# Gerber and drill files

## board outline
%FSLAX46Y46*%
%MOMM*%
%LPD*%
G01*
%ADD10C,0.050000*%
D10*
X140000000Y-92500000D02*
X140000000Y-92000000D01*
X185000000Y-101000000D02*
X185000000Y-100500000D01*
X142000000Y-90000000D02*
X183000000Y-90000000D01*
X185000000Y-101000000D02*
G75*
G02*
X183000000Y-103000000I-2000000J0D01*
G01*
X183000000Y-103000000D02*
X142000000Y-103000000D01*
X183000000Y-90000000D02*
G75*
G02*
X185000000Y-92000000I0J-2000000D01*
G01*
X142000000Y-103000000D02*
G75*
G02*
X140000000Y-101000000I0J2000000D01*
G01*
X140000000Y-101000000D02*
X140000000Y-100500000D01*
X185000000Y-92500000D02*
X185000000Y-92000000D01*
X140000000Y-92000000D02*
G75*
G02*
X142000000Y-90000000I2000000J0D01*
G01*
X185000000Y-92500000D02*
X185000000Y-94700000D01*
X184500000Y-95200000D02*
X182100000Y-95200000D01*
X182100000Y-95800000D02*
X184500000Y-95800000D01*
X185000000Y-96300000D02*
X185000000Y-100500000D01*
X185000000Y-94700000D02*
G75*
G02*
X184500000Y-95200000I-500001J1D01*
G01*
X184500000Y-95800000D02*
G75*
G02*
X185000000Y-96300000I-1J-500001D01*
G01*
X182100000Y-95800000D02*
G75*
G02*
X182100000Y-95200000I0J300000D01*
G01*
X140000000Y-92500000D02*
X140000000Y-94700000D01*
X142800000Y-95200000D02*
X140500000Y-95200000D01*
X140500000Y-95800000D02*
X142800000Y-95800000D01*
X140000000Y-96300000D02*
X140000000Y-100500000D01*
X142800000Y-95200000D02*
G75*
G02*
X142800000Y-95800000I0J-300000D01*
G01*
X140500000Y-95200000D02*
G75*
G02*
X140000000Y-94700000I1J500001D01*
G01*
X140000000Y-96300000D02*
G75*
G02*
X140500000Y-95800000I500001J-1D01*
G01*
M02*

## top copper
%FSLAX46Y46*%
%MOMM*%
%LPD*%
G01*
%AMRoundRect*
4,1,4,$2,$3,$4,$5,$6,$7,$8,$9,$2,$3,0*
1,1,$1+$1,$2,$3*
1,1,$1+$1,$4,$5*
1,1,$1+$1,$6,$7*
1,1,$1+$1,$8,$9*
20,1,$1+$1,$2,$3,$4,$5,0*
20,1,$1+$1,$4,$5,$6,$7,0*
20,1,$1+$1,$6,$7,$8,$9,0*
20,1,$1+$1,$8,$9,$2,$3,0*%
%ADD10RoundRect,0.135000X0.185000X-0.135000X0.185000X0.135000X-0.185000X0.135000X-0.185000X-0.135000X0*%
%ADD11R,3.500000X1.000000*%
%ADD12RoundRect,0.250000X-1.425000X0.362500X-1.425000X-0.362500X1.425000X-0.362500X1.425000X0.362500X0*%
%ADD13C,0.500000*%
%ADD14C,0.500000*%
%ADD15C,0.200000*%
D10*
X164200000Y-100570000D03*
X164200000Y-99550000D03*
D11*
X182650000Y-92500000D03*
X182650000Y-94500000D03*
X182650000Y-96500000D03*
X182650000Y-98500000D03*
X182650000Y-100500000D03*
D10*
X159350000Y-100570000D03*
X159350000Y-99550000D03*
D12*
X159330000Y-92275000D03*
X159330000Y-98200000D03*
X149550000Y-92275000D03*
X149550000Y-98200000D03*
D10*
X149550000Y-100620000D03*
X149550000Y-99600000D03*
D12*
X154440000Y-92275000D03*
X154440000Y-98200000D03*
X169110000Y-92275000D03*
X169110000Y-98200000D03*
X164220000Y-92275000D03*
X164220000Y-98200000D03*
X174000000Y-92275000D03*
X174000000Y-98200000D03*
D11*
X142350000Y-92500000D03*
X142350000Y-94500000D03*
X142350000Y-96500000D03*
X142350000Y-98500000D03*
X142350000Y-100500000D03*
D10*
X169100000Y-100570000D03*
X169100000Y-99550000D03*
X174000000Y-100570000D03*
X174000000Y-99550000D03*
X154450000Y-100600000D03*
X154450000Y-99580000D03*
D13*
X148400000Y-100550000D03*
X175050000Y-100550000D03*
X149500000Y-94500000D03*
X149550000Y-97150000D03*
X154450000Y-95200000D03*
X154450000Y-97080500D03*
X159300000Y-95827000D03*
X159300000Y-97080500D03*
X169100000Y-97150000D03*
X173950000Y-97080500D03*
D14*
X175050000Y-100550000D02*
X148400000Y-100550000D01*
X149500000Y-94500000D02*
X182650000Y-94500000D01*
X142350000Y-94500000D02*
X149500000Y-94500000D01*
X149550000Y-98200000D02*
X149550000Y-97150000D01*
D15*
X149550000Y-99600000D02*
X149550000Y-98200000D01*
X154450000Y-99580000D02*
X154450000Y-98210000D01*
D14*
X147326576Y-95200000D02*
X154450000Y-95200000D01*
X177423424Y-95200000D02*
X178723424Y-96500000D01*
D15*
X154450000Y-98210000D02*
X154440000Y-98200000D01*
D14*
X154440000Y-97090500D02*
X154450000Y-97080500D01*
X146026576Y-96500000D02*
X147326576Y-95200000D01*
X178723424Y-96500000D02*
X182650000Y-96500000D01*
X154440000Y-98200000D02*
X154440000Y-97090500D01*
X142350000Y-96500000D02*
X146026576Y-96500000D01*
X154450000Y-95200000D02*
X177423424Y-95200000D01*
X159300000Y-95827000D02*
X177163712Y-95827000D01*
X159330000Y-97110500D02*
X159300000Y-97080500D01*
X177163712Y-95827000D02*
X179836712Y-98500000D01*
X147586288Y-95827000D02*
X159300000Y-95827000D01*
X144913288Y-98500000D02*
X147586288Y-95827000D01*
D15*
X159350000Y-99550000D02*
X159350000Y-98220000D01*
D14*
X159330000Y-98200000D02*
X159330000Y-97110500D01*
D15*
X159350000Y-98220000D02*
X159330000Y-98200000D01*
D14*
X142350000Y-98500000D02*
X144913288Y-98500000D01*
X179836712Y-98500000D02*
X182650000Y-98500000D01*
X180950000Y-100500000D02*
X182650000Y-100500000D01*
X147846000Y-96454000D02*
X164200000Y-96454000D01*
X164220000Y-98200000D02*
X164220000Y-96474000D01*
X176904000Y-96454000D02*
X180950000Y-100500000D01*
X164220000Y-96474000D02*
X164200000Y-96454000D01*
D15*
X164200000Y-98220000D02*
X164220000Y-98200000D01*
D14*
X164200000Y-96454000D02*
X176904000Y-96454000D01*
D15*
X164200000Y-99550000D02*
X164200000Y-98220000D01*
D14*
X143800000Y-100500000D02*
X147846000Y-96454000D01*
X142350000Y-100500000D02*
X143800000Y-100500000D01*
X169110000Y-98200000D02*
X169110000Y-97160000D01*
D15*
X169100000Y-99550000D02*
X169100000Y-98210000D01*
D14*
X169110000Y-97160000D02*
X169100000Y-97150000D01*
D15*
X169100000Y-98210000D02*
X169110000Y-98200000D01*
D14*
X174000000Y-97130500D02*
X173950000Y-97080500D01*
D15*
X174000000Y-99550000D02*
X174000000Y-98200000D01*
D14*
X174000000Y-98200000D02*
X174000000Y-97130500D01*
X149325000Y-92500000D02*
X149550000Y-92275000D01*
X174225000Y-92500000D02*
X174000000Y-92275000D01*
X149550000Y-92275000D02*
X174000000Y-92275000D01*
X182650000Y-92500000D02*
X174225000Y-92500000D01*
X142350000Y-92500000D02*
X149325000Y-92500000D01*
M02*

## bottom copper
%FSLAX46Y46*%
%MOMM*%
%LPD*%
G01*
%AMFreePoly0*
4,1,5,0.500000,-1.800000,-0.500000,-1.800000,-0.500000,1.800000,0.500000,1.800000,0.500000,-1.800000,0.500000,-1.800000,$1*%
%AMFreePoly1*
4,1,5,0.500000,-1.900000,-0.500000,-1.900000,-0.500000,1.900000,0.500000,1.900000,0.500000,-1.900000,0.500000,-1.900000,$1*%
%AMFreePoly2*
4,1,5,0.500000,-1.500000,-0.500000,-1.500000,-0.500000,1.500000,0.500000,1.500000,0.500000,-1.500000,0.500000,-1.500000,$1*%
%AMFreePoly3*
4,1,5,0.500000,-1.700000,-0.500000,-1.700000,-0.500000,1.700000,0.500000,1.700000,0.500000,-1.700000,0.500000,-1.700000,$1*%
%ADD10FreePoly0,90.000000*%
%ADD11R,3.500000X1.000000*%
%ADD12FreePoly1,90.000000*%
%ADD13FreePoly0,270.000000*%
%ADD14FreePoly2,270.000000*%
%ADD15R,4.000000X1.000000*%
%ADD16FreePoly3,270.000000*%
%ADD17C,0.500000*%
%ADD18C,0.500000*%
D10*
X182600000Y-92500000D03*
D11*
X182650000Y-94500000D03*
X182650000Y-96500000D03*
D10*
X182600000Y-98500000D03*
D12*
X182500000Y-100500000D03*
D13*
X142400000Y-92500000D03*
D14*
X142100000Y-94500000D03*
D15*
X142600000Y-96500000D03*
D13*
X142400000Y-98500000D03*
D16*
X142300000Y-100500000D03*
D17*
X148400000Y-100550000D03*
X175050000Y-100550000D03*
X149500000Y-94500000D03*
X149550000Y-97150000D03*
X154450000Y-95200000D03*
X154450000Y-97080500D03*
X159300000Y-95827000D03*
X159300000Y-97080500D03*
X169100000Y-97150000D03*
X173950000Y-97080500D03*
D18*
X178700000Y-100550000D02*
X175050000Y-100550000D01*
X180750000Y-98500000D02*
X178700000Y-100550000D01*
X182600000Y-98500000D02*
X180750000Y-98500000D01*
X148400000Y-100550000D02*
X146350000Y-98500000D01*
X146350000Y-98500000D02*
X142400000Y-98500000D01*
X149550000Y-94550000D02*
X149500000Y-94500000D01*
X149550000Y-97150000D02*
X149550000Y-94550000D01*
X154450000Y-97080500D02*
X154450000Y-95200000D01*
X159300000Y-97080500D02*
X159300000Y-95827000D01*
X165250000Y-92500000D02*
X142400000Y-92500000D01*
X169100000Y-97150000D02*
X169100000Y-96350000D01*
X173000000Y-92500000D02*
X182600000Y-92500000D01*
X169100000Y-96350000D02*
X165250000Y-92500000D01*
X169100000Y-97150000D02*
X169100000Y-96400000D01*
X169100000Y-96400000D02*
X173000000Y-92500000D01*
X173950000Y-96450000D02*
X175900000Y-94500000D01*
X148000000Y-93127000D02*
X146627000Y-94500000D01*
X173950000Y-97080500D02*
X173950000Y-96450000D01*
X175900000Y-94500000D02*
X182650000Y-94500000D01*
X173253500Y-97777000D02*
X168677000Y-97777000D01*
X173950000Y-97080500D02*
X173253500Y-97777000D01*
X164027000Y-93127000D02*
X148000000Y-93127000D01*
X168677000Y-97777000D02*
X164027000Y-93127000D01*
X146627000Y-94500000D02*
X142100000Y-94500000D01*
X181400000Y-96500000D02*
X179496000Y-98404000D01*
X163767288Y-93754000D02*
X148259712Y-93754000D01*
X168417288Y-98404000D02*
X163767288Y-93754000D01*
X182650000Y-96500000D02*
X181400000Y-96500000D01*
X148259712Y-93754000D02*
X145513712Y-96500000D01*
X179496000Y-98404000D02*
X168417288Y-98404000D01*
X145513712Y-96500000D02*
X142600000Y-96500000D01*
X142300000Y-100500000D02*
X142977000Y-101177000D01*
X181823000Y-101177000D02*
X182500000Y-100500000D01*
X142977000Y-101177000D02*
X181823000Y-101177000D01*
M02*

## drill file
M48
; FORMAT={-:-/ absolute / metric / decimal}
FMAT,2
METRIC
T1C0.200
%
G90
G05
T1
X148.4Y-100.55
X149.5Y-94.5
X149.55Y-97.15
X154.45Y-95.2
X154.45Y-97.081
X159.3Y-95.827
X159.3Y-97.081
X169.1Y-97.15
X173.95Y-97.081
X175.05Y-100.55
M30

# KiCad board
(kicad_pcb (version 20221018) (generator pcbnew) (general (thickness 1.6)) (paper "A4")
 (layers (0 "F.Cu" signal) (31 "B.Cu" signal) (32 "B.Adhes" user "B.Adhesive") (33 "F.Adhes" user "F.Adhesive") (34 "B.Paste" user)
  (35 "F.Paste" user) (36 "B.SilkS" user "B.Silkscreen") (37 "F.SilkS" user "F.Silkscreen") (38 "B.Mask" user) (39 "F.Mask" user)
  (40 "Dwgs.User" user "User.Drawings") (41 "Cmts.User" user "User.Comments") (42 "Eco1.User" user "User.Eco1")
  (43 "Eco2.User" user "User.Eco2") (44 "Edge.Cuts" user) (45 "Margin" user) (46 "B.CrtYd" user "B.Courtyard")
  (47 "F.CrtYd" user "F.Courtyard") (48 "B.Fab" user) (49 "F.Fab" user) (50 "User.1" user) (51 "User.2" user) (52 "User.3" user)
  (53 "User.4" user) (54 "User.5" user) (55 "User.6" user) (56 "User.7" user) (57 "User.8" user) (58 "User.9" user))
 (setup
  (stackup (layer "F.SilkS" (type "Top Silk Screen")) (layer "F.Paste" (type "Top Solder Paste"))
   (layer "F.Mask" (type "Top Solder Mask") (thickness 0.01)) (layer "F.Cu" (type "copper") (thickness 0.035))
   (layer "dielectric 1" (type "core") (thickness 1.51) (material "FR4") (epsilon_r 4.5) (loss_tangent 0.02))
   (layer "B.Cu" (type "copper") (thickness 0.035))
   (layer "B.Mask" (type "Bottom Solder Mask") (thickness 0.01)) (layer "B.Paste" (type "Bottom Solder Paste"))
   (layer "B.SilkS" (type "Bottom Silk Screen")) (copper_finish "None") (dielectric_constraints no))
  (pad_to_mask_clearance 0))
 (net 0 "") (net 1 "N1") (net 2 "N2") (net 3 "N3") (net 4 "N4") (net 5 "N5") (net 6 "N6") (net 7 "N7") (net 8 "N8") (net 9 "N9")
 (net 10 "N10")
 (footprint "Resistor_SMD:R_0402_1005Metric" (layer "F.Cu") (at 164.2 100.06 90)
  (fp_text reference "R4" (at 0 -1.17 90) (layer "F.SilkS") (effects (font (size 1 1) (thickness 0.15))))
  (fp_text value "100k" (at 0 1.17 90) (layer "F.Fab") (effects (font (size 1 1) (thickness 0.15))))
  (pad "1" smd roundrect (at -0.51 0 90) (size 0.54 0.64) (layers "F.Cu" "F.Paste" "F.Mask") (roundrect_rratio 0.25) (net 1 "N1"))
  (pad "2" smd roundrect (at 0.51 0 90) (size 0.54 0.64) (layers "F.Cu" "F.Paste" "F.Mask") (roundrect_rratio 0.25) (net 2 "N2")))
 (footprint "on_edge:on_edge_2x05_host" (layer "F.Cu") (at 185 96.5 -90)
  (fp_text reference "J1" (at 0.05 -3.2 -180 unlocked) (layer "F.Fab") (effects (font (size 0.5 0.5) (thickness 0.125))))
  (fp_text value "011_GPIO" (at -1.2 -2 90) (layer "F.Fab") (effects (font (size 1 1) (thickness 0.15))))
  (fp_line (start -4 0) (end -1.8 0) (stroke (width 0.05) (type solid)) (layer "Edge.Cuts"))
  (fp_line (start -1.3 0.5) (end -1.3 2.9) (stroke (width 0.05) (type solid)) (layer "Edge.Cuts"))
  (fp_line (start -0.7 2.9) (end -0.7 0.5) (stroke (width 0.05) (type solid)) (layer "Edge.Cuts"))
  (fp_line (start -0.2 0) (end 4 0) (stroke (width 0.05) (type solid)) (layer "Edge.Cuts"))
  (fp_arc (start -1.8 0) (mid -1.446447 0.146447) (end -1.3 0.5) (stroke (width 0.05) (type solid)) (layer "Edge.Cuts"))
  (fp_arc (start -0.7 0.5) (mid -0.553553 0.146447) (end -0.2 0) (stroke (width 0.05) (type solid)) (layer "Edge.Cuts"))
  (fp_arc (start -0.7 2.9) (mid -1 3.2) (end -1.3 2.9) (stroke (width 0.05) (type solid)) (layer "Edge.Cuts"))
  (pad "1" smd rect (at -4 2.35 270) (size 1 3.5) (layers "F.Cu" "F.Mask") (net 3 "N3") (zone_connect 0))
  (pad "2" smd rect (at -2 2.35 270) (size 1 3.5) (layers "F.Cu" "F.Mask") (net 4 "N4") (zone_connect 0))
  (pad "3" smd rect (at 0 2.35 270) (size 1 3.5) (layers "F.Cu" "F.Mask") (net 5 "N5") (zone_connect 0))
  (pad "4" smd rect (at 2 2.35 270) (size 1 3.5) (layers "F.Cu" "F.Mask") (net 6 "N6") (zone_connect 0))
  (pad "5" smd rect (at 4 2.35 270) (size 1 3.5) (layers "F.Cu" "F.Mask") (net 2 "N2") (zone_connect 0))
  (pad "6" smd custom (at -4 2.4 90) (size 1 3.6) (layers "B.Cu" "B.Mask") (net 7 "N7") (zone_connect 0)
   (options (clearance outline) (anchor rect)) (primitives))
  (pad "7" smd rect (at -2 2.35 90) (size 1 3.5) (layers "B.Cu" "B.Mask") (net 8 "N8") (zone_connect 0))
  (pad "8" smd rect (at 0 2.35 90) (size 1 3.5) (layers "B.Cu" "B.Mask") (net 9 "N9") (zone_connect 0))
  (pad "9" smd custom (at 2 2.4 90) (size 1 3.6) (layers "B.Cu" "B.Mask") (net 1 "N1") (zone_connect 0)
   (options (clearance outline) (anchor rect)) (primitives))
  (pad "10" smd custom (at 4 2.5 90) (size 1 3.8) (layers "B.Cu" "B.Mask") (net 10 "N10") (zone_connect 0)
   (options (clearance outline) (anchor rect)) (primitives))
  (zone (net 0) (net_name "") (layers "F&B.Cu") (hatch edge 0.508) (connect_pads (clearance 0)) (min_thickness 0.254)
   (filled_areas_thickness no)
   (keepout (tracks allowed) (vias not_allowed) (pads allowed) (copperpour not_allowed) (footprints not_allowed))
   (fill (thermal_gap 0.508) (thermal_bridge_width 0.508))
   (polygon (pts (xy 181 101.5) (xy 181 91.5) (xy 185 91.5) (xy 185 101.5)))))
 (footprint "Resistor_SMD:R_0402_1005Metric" (layer "F.Cu") (at 159.35 100.06 90)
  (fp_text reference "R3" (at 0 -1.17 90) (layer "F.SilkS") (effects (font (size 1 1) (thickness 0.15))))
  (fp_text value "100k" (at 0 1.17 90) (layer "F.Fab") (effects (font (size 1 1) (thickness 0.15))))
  (pad "1" smd roundrect (at -0.51 0 90) (size 0.54 0.64) (layers "F.Cu" "F.Paste" "F.Mask") (roundrect_rratio 0.25) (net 1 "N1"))
  (pad "2" smd roundrect (at 0.51 0 90) (size 0.54 0.64) (layers "F.Cu" "F.Paste" "F.Mask") (roundrect_rratio 0.25) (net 6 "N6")))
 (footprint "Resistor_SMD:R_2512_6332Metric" (layer "F.Cu") (at 159.33 95.2375 -90)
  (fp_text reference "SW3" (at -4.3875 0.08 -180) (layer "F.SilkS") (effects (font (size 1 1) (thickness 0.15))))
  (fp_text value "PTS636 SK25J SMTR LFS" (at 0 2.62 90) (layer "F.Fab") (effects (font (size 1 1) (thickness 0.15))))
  (pad "1" smd roundrect (at -2.9625 0 270) (size 1.225 3.35) (layers "F.Cu" "F.Paste" "F.Mask") (roundrect_rratio 0.2040816327)
   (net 3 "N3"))
  (pad "2" smd roundrect (at 2.9625 0 270) (size 1.225 3.35) (layers "F.Cu" "F.Paste" "F.Mask") (roundrect_rratio 0.2040816327) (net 6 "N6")))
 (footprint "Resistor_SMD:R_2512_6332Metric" (layer "F.Cu") (at 149.55 95.2375 -90)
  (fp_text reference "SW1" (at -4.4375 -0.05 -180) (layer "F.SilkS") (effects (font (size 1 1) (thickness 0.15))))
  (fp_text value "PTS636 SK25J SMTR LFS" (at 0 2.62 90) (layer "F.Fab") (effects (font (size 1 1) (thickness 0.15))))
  (pad "1" smd roundrect (at -2.9625 0 270) (size 1.225 3.35) (layers "F.Cu" "F.Paste" "F.Mask") (roundrect_rratio 0.2040816327)
   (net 3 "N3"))
  (pad "2" smd roundrect (at 2.9625 0 270) (size 1.225 3.35) (layers "F.Cu" "F.Paste" "F.Mask") (roundrect_rratio 0.2040816327) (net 4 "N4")))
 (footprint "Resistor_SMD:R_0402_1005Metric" (layer "F.Cu") (at 149.55 100.11 90)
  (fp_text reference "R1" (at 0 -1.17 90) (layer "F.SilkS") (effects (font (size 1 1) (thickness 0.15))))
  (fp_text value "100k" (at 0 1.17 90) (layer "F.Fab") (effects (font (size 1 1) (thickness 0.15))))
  (pad "1" smd roundrect (at -0.51 0 90) (size 0.54 0.64) (layers "F.Cu" "F.Paste" "F.Mask") (roundrect_rratio 0.25) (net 1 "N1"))
  (pad "2" smd roundrect (at 0.51 0 90) (size 0.54 0.64) (layers "F.Cu" "F.Paste" "F.Mask") (roundrect_rratio 0.25) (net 4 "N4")))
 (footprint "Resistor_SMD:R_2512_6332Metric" (layer "F.Cu") (at 154.44 95.2375 -90)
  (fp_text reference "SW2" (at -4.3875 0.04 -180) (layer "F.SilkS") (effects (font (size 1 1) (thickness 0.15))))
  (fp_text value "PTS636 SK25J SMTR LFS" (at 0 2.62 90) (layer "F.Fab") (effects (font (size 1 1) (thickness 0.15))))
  (pad "1" smd roundrect (at -2.9625 0 270) (size 1.225 3.35) (layers "F.Cu" "F.Paste" "F.Mask") (roundrect_rratio 0.2040816327)
   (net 3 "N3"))
  (pad "2" smd roundrect (at 2.9625 0 270) (size 1.225 3.35) (layers "F.Cu" "F.Paste" "F.Mask") (roundrect_rratio 0.2040816327) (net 5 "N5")))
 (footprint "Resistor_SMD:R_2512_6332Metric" (layer "F.Cu") (at 169.11 95.2375 -90)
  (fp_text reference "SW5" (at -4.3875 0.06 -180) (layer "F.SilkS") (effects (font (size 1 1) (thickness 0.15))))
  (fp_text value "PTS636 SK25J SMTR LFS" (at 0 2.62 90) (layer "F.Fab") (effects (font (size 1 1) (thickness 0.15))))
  (pad "1" smd roundrect (at -2.9625 0 270) (size 1.225 3.35) (layers "F.Cu" "F.Paste" "F.Mask") (roundrect_rratio 0.2040816327)
   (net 3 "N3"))
  (pad "2" smd roundrect (at 2.9625 0 270) (size 1.225 3.35) (layers "F.Cu" "F.Paste" "F.Mask") (roundrect_rratio 0.2040816327) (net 7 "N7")))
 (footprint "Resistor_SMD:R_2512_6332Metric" (layer "F.Cu") (at 164.22 95.2375 -90)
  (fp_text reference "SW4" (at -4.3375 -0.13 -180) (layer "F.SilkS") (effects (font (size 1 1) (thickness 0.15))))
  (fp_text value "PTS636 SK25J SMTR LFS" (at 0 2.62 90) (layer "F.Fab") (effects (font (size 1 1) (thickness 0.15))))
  (pad "1" smd roundrect (at -2.9625 0 270) (size 1.225 3.35) (layers "F.Cu" "F.Paste" "F.Mask") (roundrect_rratio 0.2040816327)
   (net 3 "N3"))
  (pad "2" smd roundrect (at 2.9625 0 270) (size 1.225 3.35) (layers "F.Cu" "F.Paste" "F.Mask") (roundrect_rratio 0.2040816327) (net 2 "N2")))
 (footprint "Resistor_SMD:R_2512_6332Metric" (layer "F.Cu") (at 174 95.2375 -90)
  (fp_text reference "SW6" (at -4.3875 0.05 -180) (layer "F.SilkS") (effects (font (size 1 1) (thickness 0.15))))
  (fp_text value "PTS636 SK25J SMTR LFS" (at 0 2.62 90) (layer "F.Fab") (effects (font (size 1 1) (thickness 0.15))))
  (pad "1" smd roundrect (at -2.9625 0 270) (size 1.225 3.35) (layers "F.Cu" "F.Paste" "F.Mask") (roundrect_rratio 0.2040816327)
   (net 3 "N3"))
  (pad "2" smd roundrect (at 2.9625 0 270) (size 1.225 3.35) (layers "F.Cu" "F.Paste" "F.Mask") (roundrect_rratio 0.2040816327) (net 8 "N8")))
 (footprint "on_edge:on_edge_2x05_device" (layer "F.Cu") (at 140 96.5 -90)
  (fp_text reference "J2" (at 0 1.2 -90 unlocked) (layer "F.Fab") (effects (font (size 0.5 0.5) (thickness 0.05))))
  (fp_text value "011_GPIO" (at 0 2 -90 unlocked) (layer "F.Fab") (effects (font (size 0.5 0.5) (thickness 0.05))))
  (fp_line (start -4 0) (end -1.8 0) (stroke (width 0.05) (type solid)) (layer "Edge.Cuts"))
  (fp_line (start -1.3 -2.8) (end -1.3 -0.5) (stroke (width 0.05) (type solid)) (layer "Edge.Cuts"))
  (fp_line (start -0.7 -0.5) (end -0.7 -2.8) (stroke (width 0.05) (type solid)) (layer "Edge.Cuts"))
  (fp_line (start -0.2 0) (end 4 0) (stroke (width 0.05) (type solid)) (layer "Edge.Cuts"))
  (fp_arc (start -1.3 -2.8) (mid -1 -3.1) (end -0.7 -2.8) (stroke (width 0.05) (type solid)) (layer "Edge.Cuts"))
  (fp_arc (start -1.3 -0.5) (mid -1.446447 -0.146447) (end -1.8 0) (stroke (width 0.05) (type solid)) (layer "Edge.Cuts"))
  (fp_arc (start -0.2 0) (mid -0.553553 -0.146447) (end -0.7 -0.5) (stroke (width 0.05) (type solid)) (layer "Edge.Cuts"))
  (pad "1" smd rect (at -4 -2.35 90) (size 1 3.5) (layers "F.Cu" "F.Mask") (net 3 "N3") (zone_connect 0))
  (pad "2" smd rect (at -2 -2.35 270) (size 1 3.5) (layers "F.Cu" "F.Mask") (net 4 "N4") (zone_connect 0))
  (pad "3" smd rect (at 0 -2.35 270) (size 1 3.5) (layers "F.Cu" "F.Mask") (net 5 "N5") (zone_connect 0))
  (pad "4" smd rect (at 2 -2.35 90) (size 1 3.5) (layers "F.Cu" "F.Mask") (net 6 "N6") (zone_connect 0))
  (pad "5" smd rect (at 4 -2.35 90) (size 1 3.5) (layers "F.Cu" "F.Mask") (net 2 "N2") (zone_connect 0))
  (pad "6" smd custom (at -4 -2.4 270) (size 1 3.6) (layers "B.Cu" "B.Mask") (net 7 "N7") (zone_connect 0)
   (options (clearance outline) (anchor rect)) (primitives))
  (pad "7" smd custom (at -2 -2.1 270) (size 1 3) (layers "B.Cu" "B.Mask") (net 8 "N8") (zone_connect 0)
   (options (clearance outline) (anchor rect)) (primitives))
  (pad "8" smd rect (at 0 -2.6 270) (size 1 4) (layers "B.Cu" "B.Mask") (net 9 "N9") (zone_connect 0))
  (pad "9" smd custom (at 2 -2.4 270) (size 1 3.6) (layers "B.Cu" "B.Mask") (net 1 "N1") (zone_connect 0)
   (options (clearance outline) (anchor rect)) (primitives))
  (pad "10" smd custom (at 4 -2.3 270) (size 1 3.4) (layers "B.Cu" "B.Mask") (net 10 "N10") (zone_connect 0)
   (options (clearance outline) (anchor rect)) (primitives))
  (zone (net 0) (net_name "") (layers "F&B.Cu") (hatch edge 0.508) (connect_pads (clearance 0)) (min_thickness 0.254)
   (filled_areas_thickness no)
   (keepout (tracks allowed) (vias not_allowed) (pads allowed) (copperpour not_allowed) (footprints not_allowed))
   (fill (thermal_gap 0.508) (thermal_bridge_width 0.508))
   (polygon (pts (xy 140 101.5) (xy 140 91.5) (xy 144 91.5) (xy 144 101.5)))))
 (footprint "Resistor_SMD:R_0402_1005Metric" (layer "F.Cu") (at 169.1 100.06 90)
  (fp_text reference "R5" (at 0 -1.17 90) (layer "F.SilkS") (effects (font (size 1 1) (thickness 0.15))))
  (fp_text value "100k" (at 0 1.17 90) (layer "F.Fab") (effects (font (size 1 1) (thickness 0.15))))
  (pad "1" smd roundrect (at -0.51 0 90) (size 0.54 0.64) (layers "F.Cu" "F.Paste" "F.Mask") (roundrect_rratio 0.25) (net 1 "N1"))
  (pad "2" smd roundrect (at 0.51 0 90) (size 0.54 0.64) (layers "F.Cu" "F.Paste" "F.Mask") (roundrect_rratio 0.25) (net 7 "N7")))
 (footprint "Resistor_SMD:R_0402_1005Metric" (layer "F.Cu") (at 174 100.06 90)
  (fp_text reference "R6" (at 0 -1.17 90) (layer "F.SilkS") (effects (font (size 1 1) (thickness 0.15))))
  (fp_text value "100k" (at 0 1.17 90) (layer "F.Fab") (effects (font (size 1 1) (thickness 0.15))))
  (pad "1" smd roundrect (at -0.51 0 90) (size 0.54 0.64) (layers "F.Cu" "F.Paste" "F.Mask") (roundrect_rratio 0.25) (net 1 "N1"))
  (pad "2" smd roundrect (at 0.51 0 90) (size 0.54 0.64) (layers "F.Cu" "F.Paste" "F.Mask") (roundrect_rratio 0.25) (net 8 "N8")))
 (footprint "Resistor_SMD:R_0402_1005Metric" (layer "F.Cu") (at 154.45 100.09 90)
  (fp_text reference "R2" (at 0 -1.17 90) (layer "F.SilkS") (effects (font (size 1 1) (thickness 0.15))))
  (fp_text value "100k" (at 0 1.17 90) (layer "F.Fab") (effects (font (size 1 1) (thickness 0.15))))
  (pad "1" smd roundrect (at -0.51 0 90) (size 0.54 0.64) (layers "F.Cu" "F.Paste" "F.Mask") (roundrect_rratio 0.25) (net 1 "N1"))
  (pad "2" smd roundrect (at 0.51 0 90) (size 0.54 0.64) (layers "F.Cu" "F.Paste" "F.Mask") (roundrect_rratio 0.25) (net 5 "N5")))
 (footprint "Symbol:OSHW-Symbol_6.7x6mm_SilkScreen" (layer "B.Cu") (at 163 95.85 180)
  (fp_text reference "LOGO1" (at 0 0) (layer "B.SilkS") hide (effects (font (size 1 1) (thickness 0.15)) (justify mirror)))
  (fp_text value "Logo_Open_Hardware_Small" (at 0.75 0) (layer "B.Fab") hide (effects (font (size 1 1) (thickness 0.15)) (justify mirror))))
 (gr_line (start 140 92.5) (end 140 92) (stroke (width 0.05) (type solid)) (layer "Edge.Cuts"))
 (gr_line (start 185 101) (end 185 100.5) (stroke (width 0.05) (type solid)) (layer "Edge.Cuts"))
 (gr_line (start 142 90) (end 183 90) (stroke (width 0.05) (type solid)) (layer "Edge.Cuts"))
 (gr_arc (start 185 101) (mid 184.414214 102.414214) (end 183 103) (stroke (width 0.05) (type solid)) (layer "Edge.Cuts"))
 (gr_line (start 183 103) (end 142 103) (stroke (width 0.05) (type solid)) (layer "Edge.Cuts"))
 (gr_arc (start 183 90) (mid 184.414214 90.585786) (end 185 92) (stroke (width 0.05) (type solid)) (layer "Edge.Cuts"))
 (gr_arc (start 142 103) (mid 140.585786 102.414214) (end 140 101) (stroke (width 0.05) (type solid)) (layer "Edge.Cuts"))
 (gr_line (start 140 101) (end 140 100.5) (stroke (width 0.05) (type solid)) (layer "Edge.Cuts"))
 (gr_line (start 185 92.5) (end 185 92) (stroke (width 0.05) (type solid)) (layer "Edge.Cuts"))
 (gr_arc (start 140 92) (mid 140.585786 90.585786) (end 142 90) (stroke (width 0.05) (type solid)) (layer "Edge.Cuts"))
 (segment (start 175.05 100.55) (end 148.4 100.55) (width 0.5) (layer "F.Cu") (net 1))
 (via (at 148.4 100.55) (size 0.5) (drill 0.2) (layers "F.Cu" "B.Cu") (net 1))
 (via (at 175.05 100.55) (size 0.5) (drill 0.2) (layers "F.Cu" "B.Cu") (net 1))
 (segment (start 178.7 100.55) (end 175.05 100.55) (width 0.5) (layer "B.Cu") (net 1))
 (segment (start 180.75 98.5) (end 178.7 100.55) (width 0.5) (layer "B.Cu") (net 1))
 (segment (start 182.6 98.5) (end 180.75 98.5) (width 0.5) (layer "B.Cu") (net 1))
 (segment (start 148.4 100.55) (end 146.35 98.5) (width 0.5) (layer "B.Cu") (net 1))
 (segment (start 146.35 98.5) (end 142.4 98.5) (width 0.5) (layer "B.Cu") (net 1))
 (segment (start 149.5 94.5) (end 182.65 94.5) (width 0.5) (layer "F.Cu") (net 4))
 (segment (start 142.35 94.5) (end 149.5 94.5) (width 0.5) (layer "F.Cu") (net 4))
 (segment (start 149.55 98.2) (end 149.55 97.15) (width 0.5) (layer "F.Cu") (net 4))
 (segment (start 149.55 99.6) (end 149.55 98.2) (width 0.2) (layer "F.Cu") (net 4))
 (via (at 149.5 94.5) (size 0.5) (drill 0.2) (layers "F.Cu" "B.Cu") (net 4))
 (via (at 149.55 97.15) (size 0.5) (drill 0.2) (layers "F.Cu" "B.Cu") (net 4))
 (segment (start 149.55 94.55) (end 149.5 94.5) (width 0.5) (layer "B.Cu") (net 4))
 (segment (start 149.55 97.15) (end 149.55 94.55) (width 0.5) (layer "B.Cu") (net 4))
 (segment (start 154.45 99.58) (end 154.45 98.21) (width 0.2) (layer "F.Cu") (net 5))
 (segment (start 147.326576 95.2) (end 154.45 95.2) (width 0.5) (layer "F.Cu") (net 5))
 (segment (start 177.423424 95.2) (end 178.723424 96.5) (width 0.5) (layer "F.Cu") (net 5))
 (segment (start 154.45 98.21) (end 154.44 98.2) (width 0.2) (layer "F.Cu") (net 5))
 (segment (start 154.44 97.0905) (end 154.45 97.0805) (width 0.5) (layer "F.Cu") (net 5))
 (segment (start 146.026576 96.5) (end 147.326576 95.2) (width 0.5) (layer "F.Cu") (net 5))
 (segment (start 178.723424 96.5) (end 182.65 96.5) (width 0.5) (layer "F.Cu") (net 5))
 (segment (start 154.44 98.2) (end 154.44 97.0905) (width 0.5) (layer "F.Cu") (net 5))
 (segment (start 142.35 96.5) (end 146.026576 96.5) (width 0.5) (layer "F.Cu") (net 5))
 (segment (start 154.45 95.2) (end 177.423424 95.2) (width 0.5) (layer "F.Cu") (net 5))
 (via (at 154.45 95.2) (size 0.5) (drill 0.2) (layers "F.Cu" "B.Cu") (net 5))
 (via (at 154.45 97.0805) (size 0.5) (drill 0.2) (layers "F.Cu" "B.Cu") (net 5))
 (segment (start 154.45 97.0805) (end 154.45 95.2) (width 0.5) (layer "B.Cu") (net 5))
 (segment (start 159.3 95.827) (end 177.163712 95.827) (width 0.5) (layer "F.Cu") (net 6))
 (segment (start 159.33 97.1105) (end 159.3 97.0805) (width 0.5) (layer "F.Cu") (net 6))
 (segment (start 177.163712 95.827) (end 179.836712 98.5) (width 0.5) (layer "F.Cu") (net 6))
 (segment (start 147.586288 95.827) (end 159.3 95.827) (width 0.5) (layer "F.Cu") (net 6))
 (segment (start 144.913288 98.5) (end 147.586288 95.827) (width 0.5) (layer "F.Cu") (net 6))
 (segment (start 159.35 99.55) (end 159.35 98.22) (width 0.2) (layer "F.Cu") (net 6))
 (segment (start 159.33 98.2) (end 159.33 97.1105) (width 0.5) (layer "F.Cu") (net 6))
 (segment (start 159.35 98.22) (end 159.33 98.2) (width 0.2) (layer "F.Cu") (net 6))
 (segment (start 142.35 98.5) (end 144.913288 98.5) (width 0.5) (layer "F.Cu") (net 6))
 (segment (start 179.836712 98.5) (end 182.65 98.5) (width 0.5) (layer "F.Cu") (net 6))
 (via (at 159.3 95.827) (size 0.5) (drill 0.2) (layers "F.Cu" "B.Cu") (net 6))
 (via (at 159.3 97.0805) (size 0.5) (drill 0.2) (layers "F.Cu" "B.Cu") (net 6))
 (segment (start 159.3 97.0805) (end 159.3 95.827) (width 0.5) (layer "B.Cu") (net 6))
 (segment (start 180.95 100.5) (end 182.65 100.5) (width 0.5) (layer "F.Cu") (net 2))
 (segment (start 147.846 96.454) (end 164.2 96.454) (width 0.5) (layer "F.Cu") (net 2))
 (segment (start 164.22 98.2) (end 164.22 96.474) (width 0.5) (layer "F.Cu") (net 2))
 (segment (start 176.904 96.454) (end 180.95 100.5) (width 0.5) (layer "F.Cu") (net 2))
 (segment (start 164.22 96.474) (end 164.2 96.454) (width 0.5) (layer "F.Cu") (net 2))
 (segment (start 164.2 98.22) (end 164.22 98.2) (width 0.2) (layer "F.Cu") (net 2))
 (segment (start 164.2 96.454) (end 176.904 96.454) (width 0.5) (layer "F.Cu") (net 2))
 (segment (start 164.2 99.55) (end 164.2 98.22) (width 0.2) (layer "F.Cu") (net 2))
 (segment (start 143.8 100.5) (end 147.846 96.454) (width 0.5) (layer "F.Cu") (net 2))
 (segment (start 142.35 100.5) (end 143.8 100.5) (width 0.5) (layer "F.Cu") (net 2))
 (segment (start 169.11 98.2) (end 169.11 97.16) (width 0.5) (layer "F.Cu") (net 7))
 (segment (start 169.1 99.55) (end 169.1 98.21) (width 0.2) (layer "F.Cu") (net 7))
 (segment (start 169.11 97.16) (end 169.1 97.15) (width 0.5) (layer "F.Cu") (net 7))
 (segment (start 169.1 98.21) (end 169.11 98.2) (width 0.2) (layer "F.Cu") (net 7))
 (via (at 169.1 97.15) (size 0.5) (drill 0.2) (layers "F.Cu" "B.Cu") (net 7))
 (segment (start 165.25 92.5) (end 142.4 92.5) (width 0.5) (layer "B.Cu") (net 7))
 (segment (start 169.1 97.15) (end 169.1 96.35) (width 0.5) (layer "B.Cu") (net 7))
 (segment (start 173 92.5) (end 182.6 92.5) (width 0.5) (layer "B.Cu") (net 7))
 (segment (start 169.1 96.35) (end 165.25 92.5) (width 0.5) (layer "B.Cu") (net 7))
 (segment (start 169.1 97.15) (end 169.1 96.4) (width 0.5) (layer "B.Cu") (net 7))
 (segment (start 169.1 96.4) (end 173 92.5) (width 0.5) (layer "B.Cu") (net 7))
 (segment (start 174 97.1305) (end 173.95 97.0805) (width 0.5) (layer "F.Cu") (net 8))
 (segment (start 174 99.55) (end 174 98.2) (width 0.2) (layer "F.Cu") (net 8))
 (segment (start 174 98.2) (end 174 97.1305) (width 0.5) (layer "F.Cu") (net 8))
 (via (at 173.95 97.0805) (size 0.5) (drill 0.2) (layers "F.Cu" "B.Cu") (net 8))
 (segment (start 173.95 96.45) (end 175.9 94.5) (width 0.5) (layer "B.Cu") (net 8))
 (segment (start 148 93.127) (end 146.627 94.5) (width 0.5) (layer "B.Cu") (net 8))
 (segment (start 173.95 97.0805) (end 173.95 96.45) (width 0.5) (layer "B.Cu") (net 8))
 (segment (start 175.9 94.5) (end 182.65 94.5) (width 0.5) (layer "B.Cu") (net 8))
 (segment (start 173.2535 97.777) (end 168.677 97.777) (width 0.5) (layer "B.Cu") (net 8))
 (segment (start 173.95 97.0805) (end 173.2535 97.777) (width 0.5) (layer "B.Cu") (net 8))
 (segment (start 164.027 93.127) (end 148 93.127) (width 0.5) (layer "B.Cu") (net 8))
 (segment (start 168.677 97.777) (end 164.027 93.127) (width 0.5) (layer "B.Cu") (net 8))
 (segment (start 146.627 94.5) (end 142.1 94.5) (width 0.5) (layer "B.Cu") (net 8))
 (segment (start 149.325 92.5) (end 149.55 92.275) (width 0.5) (layer "F.Cu") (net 3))
 (segment (start 174.225 92.5) (end 174 92.275) (width 0.5) (layer "F.Cu") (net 3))
 (segment (start 149.55 92.275) (end 174 92.275) (width 0.5) (layer "F.Cu") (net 3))
 (segment (start 182.65 92.5) (end 174.225 92.5) (width 0.5) (layer "F.Cu") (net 3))
 (segment (start 142.35 92.5) (end 149.325 92.5) (width 0.5) (layer "F.Cu") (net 3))
 (segment (start 181.4 96.5) (end 179.496 98.404) (width 0.5) (layer "B.Cu") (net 9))
 (segment (start 163.767288 93.754) (end 148.259712 93.754) (width 0.5) (layer "B.Cu") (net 9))
 (segment (start 168.417288 98.404) (end 163.767288 93.754) (width 0.5) (layer "B.Cu") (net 9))
 (segment (start 182.65 96.5) (end 181.4 96.5) (width 0.5) (layer "B.Cu") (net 9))
 (segment (start 148.259712 93.754) (end 145.513712 96.5) (width 0.5) (layer "B.Cu") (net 9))
 (segment (start 179.496 98.404) (end 168.417288 98.404) (width 0.5) (layer "B.Cu") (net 9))
 (segment (start 145.513712 96.5) (end 142.6 96.5) (width 0.5) (layer "B.Cu") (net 9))
 (segment (start 142.3 100.5) (end 142.977 101.177) (width 0.5) (layer "B.Cu") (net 10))
 (segment (start 181.823 101.177) (end 182.5 100.5) (width 0.5) (layer "B.Cu") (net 10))
 (segment (start 142.977 101.177) (end 181.823 101.177) (width 0.5) (layer "B.Cu") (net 10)))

